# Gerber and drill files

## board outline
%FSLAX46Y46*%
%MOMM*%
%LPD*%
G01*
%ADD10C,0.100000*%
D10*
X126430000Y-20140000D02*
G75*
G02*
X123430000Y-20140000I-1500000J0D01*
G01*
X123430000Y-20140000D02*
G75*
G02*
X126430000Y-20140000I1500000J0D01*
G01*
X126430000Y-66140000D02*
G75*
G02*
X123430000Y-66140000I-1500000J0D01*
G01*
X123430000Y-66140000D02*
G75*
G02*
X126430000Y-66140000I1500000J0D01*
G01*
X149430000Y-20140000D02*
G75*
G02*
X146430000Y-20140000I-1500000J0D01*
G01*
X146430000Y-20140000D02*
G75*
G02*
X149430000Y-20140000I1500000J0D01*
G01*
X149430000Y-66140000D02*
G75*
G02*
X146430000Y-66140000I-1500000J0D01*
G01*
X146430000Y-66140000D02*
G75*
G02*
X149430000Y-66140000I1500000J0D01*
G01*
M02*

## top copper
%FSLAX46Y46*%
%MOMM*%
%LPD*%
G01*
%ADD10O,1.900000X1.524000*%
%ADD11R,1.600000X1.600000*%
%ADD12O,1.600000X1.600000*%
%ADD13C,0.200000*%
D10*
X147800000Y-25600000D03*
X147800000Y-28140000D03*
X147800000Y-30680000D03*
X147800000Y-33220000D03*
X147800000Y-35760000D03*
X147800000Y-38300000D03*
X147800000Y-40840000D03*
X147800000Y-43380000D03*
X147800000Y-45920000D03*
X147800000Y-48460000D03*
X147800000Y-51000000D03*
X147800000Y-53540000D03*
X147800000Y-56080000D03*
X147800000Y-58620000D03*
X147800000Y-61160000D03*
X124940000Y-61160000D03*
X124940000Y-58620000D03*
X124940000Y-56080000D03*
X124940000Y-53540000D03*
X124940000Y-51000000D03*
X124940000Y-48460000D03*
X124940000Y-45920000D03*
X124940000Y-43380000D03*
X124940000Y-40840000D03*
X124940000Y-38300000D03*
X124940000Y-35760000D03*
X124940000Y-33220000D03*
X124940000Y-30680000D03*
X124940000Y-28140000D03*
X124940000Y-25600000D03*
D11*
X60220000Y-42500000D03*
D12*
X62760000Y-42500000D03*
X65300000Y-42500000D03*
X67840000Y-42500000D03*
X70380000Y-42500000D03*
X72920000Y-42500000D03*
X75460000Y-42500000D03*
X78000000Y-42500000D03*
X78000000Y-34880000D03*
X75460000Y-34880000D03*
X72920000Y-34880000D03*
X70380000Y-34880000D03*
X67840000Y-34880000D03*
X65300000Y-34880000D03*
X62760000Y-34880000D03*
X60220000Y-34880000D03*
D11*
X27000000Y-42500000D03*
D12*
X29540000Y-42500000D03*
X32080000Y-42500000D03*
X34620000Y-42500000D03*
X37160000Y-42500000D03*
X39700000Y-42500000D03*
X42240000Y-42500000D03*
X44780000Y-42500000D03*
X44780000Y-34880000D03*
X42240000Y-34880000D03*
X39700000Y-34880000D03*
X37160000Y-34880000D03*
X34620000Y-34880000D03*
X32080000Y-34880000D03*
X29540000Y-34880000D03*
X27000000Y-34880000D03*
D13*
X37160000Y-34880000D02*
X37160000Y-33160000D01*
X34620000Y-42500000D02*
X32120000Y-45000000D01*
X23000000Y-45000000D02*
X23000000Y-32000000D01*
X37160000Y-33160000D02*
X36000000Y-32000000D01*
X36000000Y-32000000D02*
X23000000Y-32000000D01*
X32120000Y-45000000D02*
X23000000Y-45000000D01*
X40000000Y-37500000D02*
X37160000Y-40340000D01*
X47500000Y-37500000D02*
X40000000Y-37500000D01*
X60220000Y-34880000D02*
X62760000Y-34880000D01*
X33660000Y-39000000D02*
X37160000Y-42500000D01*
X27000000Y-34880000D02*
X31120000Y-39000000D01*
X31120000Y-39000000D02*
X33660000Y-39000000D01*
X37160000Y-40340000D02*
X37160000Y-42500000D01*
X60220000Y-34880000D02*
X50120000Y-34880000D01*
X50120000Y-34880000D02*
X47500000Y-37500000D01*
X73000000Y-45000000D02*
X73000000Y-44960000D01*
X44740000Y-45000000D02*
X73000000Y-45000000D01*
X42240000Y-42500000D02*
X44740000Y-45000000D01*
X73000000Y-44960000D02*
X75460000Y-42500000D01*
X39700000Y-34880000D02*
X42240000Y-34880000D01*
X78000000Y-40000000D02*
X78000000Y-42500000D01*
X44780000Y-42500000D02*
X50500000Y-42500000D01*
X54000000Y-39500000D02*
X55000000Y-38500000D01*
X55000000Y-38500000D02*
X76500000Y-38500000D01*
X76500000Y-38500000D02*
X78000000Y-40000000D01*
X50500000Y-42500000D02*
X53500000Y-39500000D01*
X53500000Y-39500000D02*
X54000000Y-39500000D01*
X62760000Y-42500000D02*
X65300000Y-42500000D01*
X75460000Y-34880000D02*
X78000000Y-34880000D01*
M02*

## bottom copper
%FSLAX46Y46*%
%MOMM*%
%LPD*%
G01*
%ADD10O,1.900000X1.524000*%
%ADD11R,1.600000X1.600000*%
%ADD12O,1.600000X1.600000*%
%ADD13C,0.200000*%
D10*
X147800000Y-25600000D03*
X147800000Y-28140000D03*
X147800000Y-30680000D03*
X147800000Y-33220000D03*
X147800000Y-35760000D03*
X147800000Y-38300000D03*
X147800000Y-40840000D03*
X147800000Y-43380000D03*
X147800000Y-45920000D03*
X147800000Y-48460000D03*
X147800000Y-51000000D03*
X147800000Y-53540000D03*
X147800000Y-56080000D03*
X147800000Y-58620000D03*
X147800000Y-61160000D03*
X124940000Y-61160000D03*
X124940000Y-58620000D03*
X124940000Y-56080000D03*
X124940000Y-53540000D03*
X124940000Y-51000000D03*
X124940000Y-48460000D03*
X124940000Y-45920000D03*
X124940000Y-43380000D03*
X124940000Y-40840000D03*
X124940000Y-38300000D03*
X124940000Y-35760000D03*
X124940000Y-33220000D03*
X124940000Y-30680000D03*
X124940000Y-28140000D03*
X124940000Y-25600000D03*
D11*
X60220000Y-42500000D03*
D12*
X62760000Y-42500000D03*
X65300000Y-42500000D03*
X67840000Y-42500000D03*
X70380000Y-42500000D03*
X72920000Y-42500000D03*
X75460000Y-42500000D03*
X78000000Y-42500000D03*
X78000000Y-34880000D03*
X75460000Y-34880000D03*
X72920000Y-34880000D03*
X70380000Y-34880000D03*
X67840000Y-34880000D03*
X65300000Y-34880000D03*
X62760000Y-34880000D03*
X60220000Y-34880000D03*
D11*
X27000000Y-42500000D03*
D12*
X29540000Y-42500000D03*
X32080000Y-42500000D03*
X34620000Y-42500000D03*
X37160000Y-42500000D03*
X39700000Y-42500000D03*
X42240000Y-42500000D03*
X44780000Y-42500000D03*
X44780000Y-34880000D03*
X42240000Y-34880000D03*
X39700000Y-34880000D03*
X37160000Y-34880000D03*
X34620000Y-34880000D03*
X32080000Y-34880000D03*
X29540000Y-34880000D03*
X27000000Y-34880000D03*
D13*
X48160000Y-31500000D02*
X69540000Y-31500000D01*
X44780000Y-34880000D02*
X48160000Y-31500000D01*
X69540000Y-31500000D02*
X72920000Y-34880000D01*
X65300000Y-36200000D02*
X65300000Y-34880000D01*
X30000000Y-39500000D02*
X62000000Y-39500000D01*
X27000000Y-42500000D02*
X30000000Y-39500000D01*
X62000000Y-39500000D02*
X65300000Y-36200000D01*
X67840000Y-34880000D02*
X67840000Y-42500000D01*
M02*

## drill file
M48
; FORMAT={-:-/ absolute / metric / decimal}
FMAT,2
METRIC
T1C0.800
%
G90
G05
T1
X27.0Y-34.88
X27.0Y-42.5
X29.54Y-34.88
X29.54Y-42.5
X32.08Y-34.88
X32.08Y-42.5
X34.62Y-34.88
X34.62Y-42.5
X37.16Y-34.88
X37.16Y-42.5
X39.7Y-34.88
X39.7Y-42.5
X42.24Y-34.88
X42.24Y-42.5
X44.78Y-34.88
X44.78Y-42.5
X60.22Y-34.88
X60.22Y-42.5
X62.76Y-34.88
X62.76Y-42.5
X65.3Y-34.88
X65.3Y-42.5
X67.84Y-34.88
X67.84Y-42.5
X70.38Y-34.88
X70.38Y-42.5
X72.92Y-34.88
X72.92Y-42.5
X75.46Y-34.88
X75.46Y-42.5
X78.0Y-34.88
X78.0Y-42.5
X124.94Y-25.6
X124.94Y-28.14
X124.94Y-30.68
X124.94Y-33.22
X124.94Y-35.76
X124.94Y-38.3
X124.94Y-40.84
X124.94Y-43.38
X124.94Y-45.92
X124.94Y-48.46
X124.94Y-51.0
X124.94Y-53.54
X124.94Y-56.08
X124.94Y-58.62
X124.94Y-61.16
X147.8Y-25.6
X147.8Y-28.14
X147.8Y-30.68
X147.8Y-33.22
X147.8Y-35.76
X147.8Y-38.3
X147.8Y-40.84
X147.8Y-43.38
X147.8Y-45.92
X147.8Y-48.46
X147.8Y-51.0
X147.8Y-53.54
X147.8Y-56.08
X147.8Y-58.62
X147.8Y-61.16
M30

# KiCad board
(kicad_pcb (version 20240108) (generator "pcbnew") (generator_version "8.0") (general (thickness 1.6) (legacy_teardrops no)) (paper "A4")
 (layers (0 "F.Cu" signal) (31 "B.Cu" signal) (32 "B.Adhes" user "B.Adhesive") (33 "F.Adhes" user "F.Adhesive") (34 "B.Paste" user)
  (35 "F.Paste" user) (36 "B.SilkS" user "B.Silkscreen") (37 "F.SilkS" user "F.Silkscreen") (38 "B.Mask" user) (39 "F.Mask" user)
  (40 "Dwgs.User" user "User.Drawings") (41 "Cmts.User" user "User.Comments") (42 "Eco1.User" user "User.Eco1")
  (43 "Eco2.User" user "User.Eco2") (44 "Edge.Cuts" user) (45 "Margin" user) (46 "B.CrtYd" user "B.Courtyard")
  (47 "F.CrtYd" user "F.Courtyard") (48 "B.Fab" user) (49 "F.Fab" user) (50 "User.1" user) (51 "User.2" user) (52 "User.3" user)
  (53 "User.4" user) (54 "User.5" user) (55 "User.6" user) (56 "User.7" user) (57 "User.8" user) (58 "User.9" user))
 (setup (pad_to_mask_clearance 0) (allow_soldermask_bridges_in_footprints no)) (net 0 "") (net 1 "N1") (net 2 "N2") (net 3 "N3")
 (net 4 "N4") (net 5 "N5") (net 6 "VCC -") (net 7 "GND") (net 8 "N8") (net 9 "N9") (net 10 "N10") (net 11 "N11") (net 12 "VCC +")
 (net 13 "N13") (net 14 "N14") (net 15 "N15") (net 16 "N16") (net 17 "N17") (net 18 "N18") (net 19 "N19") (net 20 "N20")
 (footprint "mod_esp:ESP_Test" (layer "F.Cu") (at 136.5 43 -90)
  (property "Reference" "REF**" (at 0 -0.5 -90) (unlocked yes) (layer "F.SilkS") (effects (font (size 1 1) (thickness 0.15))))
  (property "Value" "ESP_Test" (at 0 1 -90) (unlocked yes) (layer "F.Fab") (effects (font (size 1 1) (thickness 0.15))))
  (fp_circle (center -22.86 11.57) (end -21.36 11.57) (stroke (width 0.1) (type default)) (fill none) (layer "Edge.Cuts"))
  (fp_circle (center 23.14 11.57) (end 24.64 11.57) (stroke (width 0.1) (type default)) (fill none) (layer "Edge.Cuts"))
  (fp_circle (center -22.86 -11.43) (end -21.36 -11.43) (stroke (width 0.1) (type default)) (fill none) (layer "Edge.Cuts"))
  (fp_circle (center 23.14 -11.43) (end 24.64 -11.43) (stroke (width 0.1) (type default)) (fill none) (layer "Edge.Cuts"))
  (pad "1" thru_hole oval (at -17.4 -11.3 270) (size 1.524 1.9) (drill 0.8) (layers "*.Cu" "*.Mask") (remove_unused_layers no))
  (pad "2" thru_hole oval (at -14.86 -11.3 270) (size 1.524 1.9) (drill 0.8) (layers "*.Cu" "*.Mask") (remove_unused_layers no))
  (pad "3" thru_hole oval (at -12.32 -11.3 270) (size 1.524 1.9) (drill 0.8) (layers "*.Cu" "*.Mask") (remove_unused_layers no))
  (pad "4" thru_hole oval (at -9.78 -11.3 270) (size 1.524 1.9) (drill 0.8) (layers "*.Cu" "*.Mask") (remove_unused_layers no))
  (pad "5" thru_hole oval (at -7.24 -11.3 270) (size 1.524 1.9) (drill 0.8) (layers "*.Cu" "*.Mask") (remove_unused_layers no))
  (pad "6" thru_hole oval (at -4.7 -11.3 270) (size 1.524 1.9) (drill 0.8) (layers "*.Cu" "*.Mask") (remove_unused_layers no))
  (pad "7" thru_hole oval (at -2.16 -11.3 270) (size 1.524 1.9) (drill 0.8) (layers "*.Cu" "*.Mask") (remove_unused_layers no))
  (pad "8" thru_hole oval (at 0.38 -11.3 270) (size 1.524 1.9) (drill 0.8) (layers "*.Cu" "*.Mask") (remove_unused_layers no))
  (pad "9" thru_hole oval (at 2.92 -11.3 270) (size 1.524 1.9) (drill 0.8) (layers "*.Cu" "*.Mask") (remove_unused_layers no))
  (pad "10" thru_hole oval (at 5.46 -11.3 270) (size 1.524 1.9) (drill 0.8) (layers "*.Cu" "*.Mask") (remove_unused_layers no))
  (pad "11" thru_hole oval (at 8 -11.3 270) (size 1.524 1.9) (drill 0.8) (layers "*.Cu" "*.Mask") (remove_unused_layers no))
  (pad "12" thru_hole oval (at 10.54 -11.3 270) (size 1.524 1.9) (drill 0.8) (layers "*.Cu" "*.Mask") (remove_unused_layers no))
  (pad "13" thru_hole oval (at 13.08 -11.3 270) (size 1.524 1.9) (drill 0.8) (layers "*.Cu" "*.Mask") (remove_unused_layers no))
  (pad "14" thru_hole oval (at 15.62 -11.3 270) (size 1.524 1.9) (drill 0.8) (layers "*.Cu" "*.Mask") (remove_unused_layers no))
  (pad "15" thru_hole oval (at 18.16 -11.3 270) (size 1.524 1.9) (drill 0.8) (layers "*.Cu" "*.Mask") (remove_unused_layers no))
  (pad "16" thru_hole oval (at 18.16 11.56 270) (size 1.524 1.9) (drill 0.8) (layers "*.Cu" "*.Mask") (remove_unused_layers no))
  (pad "17" thru_hole oval (at 15.62 11.56 270) (size 1.524 1.9) (drill 0.8) (layers "*.Cu" "*.Mask") (remove_unused_layers no))
  (pad "18" thru_hole oval (at 13.08 11.56 270) (size 1.524 1.9) (drill 0.8) (layers "*.Cu" "*.Mask") (remove_unused_layers no))
  (pad "19" thru_hole oval (at 10.54 11.56 270) (size 1.524 1.9) (drill 0.8) (layers "*.Cu" "*.Mask") (remove_unused_layers no))
  (pad "20" thru_hole oval (at 8 11.56 270) (size 1.524 1.9) (drill 0.8) (layers "*.Cu" "*.Mask") (remove_unused_layers no))
  (pad "21" thru_hole oval (at 5.46 11.56 270) (size 1.524 1.9) (drill 0.8) (layers "*.Cu" "*.Mask") (remove_unused_layers no))
  (pad "22" thru_hole oval (at 2.92 11.56 270) (size 1.524 1.9) (drill 0.8) (layers "*.Cu" "*.Mask") (remove_unused_layers no))
  (pad "23" thru_hole oval (at 0.38 11.56 270) (size 1.524 1.9) (drill 0.8) (layers "*.Cu" "*.Mask") (remove_unused_layers no))
  (pad "24" thru_hole oval (at -2.16 11.56 270) (size 1.524 1.9) (drill 0.8) (layers "*.Cu" "*.Mask") (remove_unused_layers no))
  (pad "25" thru_hole oval (at -4.7 11.56 270) (size 1.524 1.9) (drill 0.8) (layers "*.Cu" "*.Mask") (remove_unused_layers no))
  (pad "26" thru_hole oval (at -7.24 11.56 270) (size 1.524 1.9) (drill 0.8) (layers "*.Cu" "*.Mask") (remove_unused_layers no))
  (pad "27" thru_hole oval (at -9.78 11.56 270) (size 1.524 1.9) (drill 0.8) (layers "*.Cu" "*.Mask") (remove_unused_layers no))
  (pad "28" thru_hole oval (at -12.32 11.56 270) (size 1.524 1.9) (drill 0.8) (layers "*.Cu" "*.Mask") (remove_unused_layers no))
  (pad "29" thru_hole oval (at -14.86 11.56 270) (size 1.524 1.9) (drill 0.8) (layers "*.Cu" "*.Mask") (remove_unused_layers no))
  (pad "30" thru_hole oval (at -17.4 11.56 270) (size 1.524 1.9) (drill 0.8) (layers "*.Cu" "*.Mask") (remove_unused_layers no)))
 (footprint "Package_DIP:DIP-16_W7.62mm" (layer "F.Cu") (at 60.22 42.5 90)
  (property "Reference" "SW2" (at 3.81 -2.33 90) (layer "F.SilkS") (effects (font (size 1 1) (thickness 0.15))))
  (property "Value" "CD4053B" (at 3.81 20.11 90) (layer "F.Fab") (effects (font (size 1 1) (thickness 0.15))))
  (pad "1" thru_hole rect (at 0 0 90) (size 1.6 1.6) (drill 0.8) (layers "*.Cu" "*.Mask") (remove_unused_layers no) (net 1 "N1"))
  (pad "2" thru_hole oval (at 0 2.54 90) (size 1.6 1.6) (drill 0.8) (layers "*.Cu" "*.Mask") (remove_unused_layers no) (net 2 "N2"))
  (pad "3" thru_hole oval (at 0 5.08 90) (size 1.6 1.6) (drill 0.8) (layers "*.Cu" "*.Mask") (remove_unused_layers no) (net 2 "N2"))
  (pad "4" thru_hole oval (at 0 7.62 90) (size 1.6 1.6) (drill 0.8) (layers "*.Cu" "*.Mask") (remove_unused_layers no) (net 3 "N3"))
  (pad "5" thru_hole oval (at 0 10.16 90) (size 1.6 1.6) (drill 0.8) (layers "*.Cu" "*.Mask") (remove_unused_layers no) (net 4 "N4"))
  (pad "6" thru_hole oval (at 0 12.7 90) (size 1.6 1.6) (drill 0.8) (layers "*.Cu" "*.Mask") (remove_unused_layers no) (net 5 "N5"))
  (pad "7" thru_hole oval (at 0 15.24 90) (size 1.6 1.6) (drill 0.8) (layers "*.Cu" "*.Mask") (remove_unused_layers no) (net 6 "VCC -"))
  (pad "8" thru_hole oval (at 0 17.78 90) (size 1.6 1.6) (drill 0.8) (layers "*.Cu" "*.Mask") (remove_unused_layers no) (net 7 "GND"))
  (pad "9" thru_hole oval (at 7.62 17.78 90) (size 1.6 1.6) (drill 0.8) (layers "*.Cu" "*.Mask") (remove_unused_layers no) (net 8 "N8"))
  (pad "10" thru_hole oval (at 7.62 15.24 90) (size 1.6 1.6) (drill 0.8) (layers "*.Cu" "*.Mask") (remove_unused_layers no) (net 8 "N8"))
  (pad "11" thru_hole oval (at 7.62 12.7 90) (size 1.6 1.6) (drill 0.8) (layers "*.Cu" "*.Mask") (remove_unused_layers no) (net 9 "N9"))
  (pad "12" thru_hole oval (at 7.62 10.16 90) (size 1.6 1.6) (drill 0.8) (layers "*.Cu" "*.Mask") (remove_unused_layers no) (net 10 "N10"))
  (pad "13" thru_hole oval (at 7.62 7.62 90) (size 1.6 1.6) (drill 0.8) (layers "*.Cu" "*.Mask") (remove_unused_layers no) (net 3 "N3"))
  (pad "14" thru_hole oval (at 7.62 5.08 90) (size 1.6 1.6) (drill 0.8) (layers "*.Cu" "*.Mask") (remove_unused_layers no) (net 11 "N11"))
  (pad "15" thru_hole oval (at 7.62 2.54 90) (size 1.6 1.6) (drill 0.8) (layers "*.Cu" "*.Mask") (remove_unused_layers no) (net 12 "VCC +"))
  (pad "16" thru_hole oval (at 7.62 0 90) (size 1.6 1.6) (drill 0.8) (layers "*.Cu" "*.Mask") (remove_unused_layers no) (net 12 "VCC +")))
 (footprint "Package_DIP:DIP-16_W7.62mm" (layer "F.Cu") (at 27 42.5 90)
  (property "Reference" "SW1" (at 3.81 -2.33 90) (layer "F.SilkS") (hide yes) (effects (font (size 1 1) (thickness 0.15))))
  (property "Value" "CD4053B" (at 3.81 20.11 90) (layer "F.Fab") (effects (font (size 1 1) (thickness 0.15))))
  (pad "1" thru_hole rect (at 0 0 90) (size 1.6 1.6) (drill 0.8) (layers "*.Cu" "*.Mask") (remove_unused_layers no) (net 11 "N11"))
  (pad "2" thru_hole oval (at 0 2.54 90) (size 1.6 1.6) (drill 0.8) (layers "*.Cu" "*.Mask") (remove_unused_layers no) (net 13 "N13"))
  (pad "3" thru_hole oval (at 0 5.08 90) (size 1.6 1.6) (drill 0.8) (layers "*.Cu" "*.Mask") (remove_unused_layers no) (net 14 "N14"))
  (pad "4" thru_hole oval (at 0 7.62 90) (size 1.6 1.6) (drill 0.8) (layers "*.Cu" "*.Mask") (remove_unused_layers no) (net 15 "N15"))
  (pad "5" thru_hole oval (at 0 10.16 90) (size 1.6 1.6) (drill 0.8) (layers "*.Cu" "*.Mask") (remove_unused_layers no) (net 12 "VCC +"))
  (pad "6" thru_hole oval (at 0 12.7 90) (size 1.6 1.6) (drill 0.8) (layers "*.Cu" "*.Mask") (remove_unused_layers no) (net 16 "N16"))
  (pad "7" thru_hole oval (at 0 15.24 90) (size 1.6 1.6) (drill 0.8) (layers "*.Cu" "*.Mask") (remove_unused_layers no) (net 6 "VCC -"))
  (pad "8" thru_hole oval (at 0 17.78 90) (size 1.6 1.6) (drill 0.8) (layers "*.Cu" "*.Mask") (remove_unused_layers no) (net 7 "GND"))
  (pad "9" thru_hole oval (at 7.62 17.78 90) (size 1.6 1.6) (drill 0.8) (layers "*.Cu" "*.Mask") (remove_unused_layers no) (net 9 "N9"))
  (pad "10" thru_hole oval (at 7.62 15.24 90) (size 1.6 1.6) (drill 0.8) (layers "*.Cu" "*.Mask") (remove_unused_layers no) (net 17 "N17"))
  (pad "11" thru_hole oval (at 7.62 12.7 90) (size 1.6 1.6) (drill 0.8) (layers "*.Cu" "*.Mask") (remove_unused_layers no) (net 17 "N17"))
  (pad "12" thru_hole oval (at 7.62 10.16 90) (size 1.6 1.6) (drill 0.8) (layers "*.Cu" "*.Mask") (remove_unused_layers no) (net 15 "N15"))
  (pad "13" thru_hole oval (at 7.62 7.62 90) (size 1.6 1.6) (drill 0.8) (layers "*.Cu" "*.Mask") (remove_unused_layers no) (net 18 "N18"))
  (pad "14" thru_hole oval (at 7.62 5.08 90) (size 1.6 1.6) (drill 0.8) (layers "*.Cu" "*.Mask") (remove_unused_layers no) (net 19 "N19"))
  (pad "15" thru_hole oval (at 7.62 2.54 90) (size 1.6 1.6) (drill 0.8) (layers "*.Cu" "*.Mask") (remove_unused_layers no) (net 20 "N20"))
  (pad "16" thru_hole oval (at 7.62 0 90) (size 1.6 1.6) (drill 0.8) (layers "*.Cu" "*.Mask") (remove_unused_layers no) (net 12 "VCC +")))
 (segment (start 37.16 34.88) (end 37.16 33.16) (width 0.2) (layer "F.Cu") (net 15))
 (segment (start 34.62 42.5) (end 32.12 45) (width 0.2) (layer "F.Cu") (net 15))
 (segment (start 23 45) (end 23 32) (width 0.2) (layer "F.Cu") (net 15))
 (segment (start 37.16 33.16) (end 36 32) (width 0.2) (layer "F.Cu") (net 15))
 (segment (start 36 32) (end 23 32) (width 0.2) (layer "F.Cu") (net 15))
 (segment (start 32.12 45) (end 23 45) (width 0.2) (layer "F.Cu") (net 15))
 (segment (start 40 37.5) (end 37.16 40.34) (width 0.2) (layer "F.Cu") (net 12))
 (segment (start 47.5 37.5) (end 40 37.5) (width 0.2) (layer "F.Cu") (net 12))
 (segment (start 60.22 34.88) (end 62.76 34.88) (width 0.2) (layer "F.Cu") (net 12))
 (segment (start 33.66 39) (end 37.16 42.5) (width 0.2) (layer "F.Cu") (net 12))
 (segment (start 27 34.88) (end 31.12 39) (width 0.2) (layer "F.Cu") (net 12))
 (segment (start 31.12 39) (end 33.66 39) (width 0.2) (layer "F.Cu") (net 12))
 (segment (start 37.16 40.34) (end 37.16 42.5) (width 0.2) (layer "F.Cu") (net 12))
 (segment (start 60.22 34.88) (end 50.12 34.88) (width 0.2) (layer "F.Cu") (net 12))
 (segment (start 50.12 34.88) (end 47.5 37.5) (width 0.2) (layer "F.Cu") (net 12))
 (segment (start 73 45) (end 73 44.96) (width 0.2) (layer "F.Cu") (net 6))
 (segment (start 44.74 45) (end 73 45) (width 0.2) (layer "F.Cu") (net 6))
 (segment (start 42.24 42.5) (end 44.74 45) (width 0.2) (layer "F.Cu") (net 6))
 (segment (start 73 44.96) (end 75.46 42.5) (width 0.2) (layer "F.Cu") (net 6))
 (segment (start 48.16 31.5) (end 69.54 31.5) (width 0.2) (layer "B.Cu") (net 9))
 (segment (start 44.78 34.88) (end 48.16 31.5) (width 0.2) (layer "B.Cu") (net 9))
 (segment (start 69.54 31.5) (end 72.92 34.88) (width 0.2) (layer "B.Cu") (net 9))
 (segment (start 39.7 34.88) (end 42.24 34.88) (width 0.2) (layer "F.Cu") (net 17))
 (segment (start 78 40) (end 78 42.5) (width 0.2) (layer "F.Cu") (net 7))
 (segment (start 44.78 42.5) (end 50.5 42.5) (width 0.2) (layer "F.Cu") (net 7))
 (segment (start 54 39.5) (end 55 38.5) (width 0.2) (layer "F.Cu") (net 7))
 (segment (start 55 38.5) (end 76.5 38.5) (width 0.2) (layer "F.Cu") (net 7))
 (segment (start 76.5 38.5) (end 78 40) (width 0.2) (layer "F.Cu") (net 7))
 (segment (start 50.5 42.5) (end 53.5 39.5) (width 0.2) (layer "F.Cu") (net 7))
 (segment (start 53.5 39.5) (end 54 39.5) (width 0.2) (layer "F.Cu") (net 7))
 (segment (start 65.3 36.2) (end 65.3 34.88) (width 0.2) (layer "B.Cu") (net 11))
 (segment (start 30 39.5) (end 62 39.5) (width 0.2) (layer "B.Cu") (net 11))
 (segment (start 27 42.5) (end 30 39.5) (width 0.2) (layer "B.Cu") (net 11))
 (segment (start 62 39.5) (end 65.3 36.2) (width 0.2) (layer "B.Cu") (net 11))
 (segment (start 67.84 34.88) (end 67.84 42.5) (width 0.2) (layer "B.Cu") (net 3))
 (segment (start 62.76 42.5) (end 65.3 42.5) (width 0.2) (layer "F.Cu") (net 2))
 (segment (start 75.46 34.88) (end 78 34.88) (width 0.2) (layer "F.Cu") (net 8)))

